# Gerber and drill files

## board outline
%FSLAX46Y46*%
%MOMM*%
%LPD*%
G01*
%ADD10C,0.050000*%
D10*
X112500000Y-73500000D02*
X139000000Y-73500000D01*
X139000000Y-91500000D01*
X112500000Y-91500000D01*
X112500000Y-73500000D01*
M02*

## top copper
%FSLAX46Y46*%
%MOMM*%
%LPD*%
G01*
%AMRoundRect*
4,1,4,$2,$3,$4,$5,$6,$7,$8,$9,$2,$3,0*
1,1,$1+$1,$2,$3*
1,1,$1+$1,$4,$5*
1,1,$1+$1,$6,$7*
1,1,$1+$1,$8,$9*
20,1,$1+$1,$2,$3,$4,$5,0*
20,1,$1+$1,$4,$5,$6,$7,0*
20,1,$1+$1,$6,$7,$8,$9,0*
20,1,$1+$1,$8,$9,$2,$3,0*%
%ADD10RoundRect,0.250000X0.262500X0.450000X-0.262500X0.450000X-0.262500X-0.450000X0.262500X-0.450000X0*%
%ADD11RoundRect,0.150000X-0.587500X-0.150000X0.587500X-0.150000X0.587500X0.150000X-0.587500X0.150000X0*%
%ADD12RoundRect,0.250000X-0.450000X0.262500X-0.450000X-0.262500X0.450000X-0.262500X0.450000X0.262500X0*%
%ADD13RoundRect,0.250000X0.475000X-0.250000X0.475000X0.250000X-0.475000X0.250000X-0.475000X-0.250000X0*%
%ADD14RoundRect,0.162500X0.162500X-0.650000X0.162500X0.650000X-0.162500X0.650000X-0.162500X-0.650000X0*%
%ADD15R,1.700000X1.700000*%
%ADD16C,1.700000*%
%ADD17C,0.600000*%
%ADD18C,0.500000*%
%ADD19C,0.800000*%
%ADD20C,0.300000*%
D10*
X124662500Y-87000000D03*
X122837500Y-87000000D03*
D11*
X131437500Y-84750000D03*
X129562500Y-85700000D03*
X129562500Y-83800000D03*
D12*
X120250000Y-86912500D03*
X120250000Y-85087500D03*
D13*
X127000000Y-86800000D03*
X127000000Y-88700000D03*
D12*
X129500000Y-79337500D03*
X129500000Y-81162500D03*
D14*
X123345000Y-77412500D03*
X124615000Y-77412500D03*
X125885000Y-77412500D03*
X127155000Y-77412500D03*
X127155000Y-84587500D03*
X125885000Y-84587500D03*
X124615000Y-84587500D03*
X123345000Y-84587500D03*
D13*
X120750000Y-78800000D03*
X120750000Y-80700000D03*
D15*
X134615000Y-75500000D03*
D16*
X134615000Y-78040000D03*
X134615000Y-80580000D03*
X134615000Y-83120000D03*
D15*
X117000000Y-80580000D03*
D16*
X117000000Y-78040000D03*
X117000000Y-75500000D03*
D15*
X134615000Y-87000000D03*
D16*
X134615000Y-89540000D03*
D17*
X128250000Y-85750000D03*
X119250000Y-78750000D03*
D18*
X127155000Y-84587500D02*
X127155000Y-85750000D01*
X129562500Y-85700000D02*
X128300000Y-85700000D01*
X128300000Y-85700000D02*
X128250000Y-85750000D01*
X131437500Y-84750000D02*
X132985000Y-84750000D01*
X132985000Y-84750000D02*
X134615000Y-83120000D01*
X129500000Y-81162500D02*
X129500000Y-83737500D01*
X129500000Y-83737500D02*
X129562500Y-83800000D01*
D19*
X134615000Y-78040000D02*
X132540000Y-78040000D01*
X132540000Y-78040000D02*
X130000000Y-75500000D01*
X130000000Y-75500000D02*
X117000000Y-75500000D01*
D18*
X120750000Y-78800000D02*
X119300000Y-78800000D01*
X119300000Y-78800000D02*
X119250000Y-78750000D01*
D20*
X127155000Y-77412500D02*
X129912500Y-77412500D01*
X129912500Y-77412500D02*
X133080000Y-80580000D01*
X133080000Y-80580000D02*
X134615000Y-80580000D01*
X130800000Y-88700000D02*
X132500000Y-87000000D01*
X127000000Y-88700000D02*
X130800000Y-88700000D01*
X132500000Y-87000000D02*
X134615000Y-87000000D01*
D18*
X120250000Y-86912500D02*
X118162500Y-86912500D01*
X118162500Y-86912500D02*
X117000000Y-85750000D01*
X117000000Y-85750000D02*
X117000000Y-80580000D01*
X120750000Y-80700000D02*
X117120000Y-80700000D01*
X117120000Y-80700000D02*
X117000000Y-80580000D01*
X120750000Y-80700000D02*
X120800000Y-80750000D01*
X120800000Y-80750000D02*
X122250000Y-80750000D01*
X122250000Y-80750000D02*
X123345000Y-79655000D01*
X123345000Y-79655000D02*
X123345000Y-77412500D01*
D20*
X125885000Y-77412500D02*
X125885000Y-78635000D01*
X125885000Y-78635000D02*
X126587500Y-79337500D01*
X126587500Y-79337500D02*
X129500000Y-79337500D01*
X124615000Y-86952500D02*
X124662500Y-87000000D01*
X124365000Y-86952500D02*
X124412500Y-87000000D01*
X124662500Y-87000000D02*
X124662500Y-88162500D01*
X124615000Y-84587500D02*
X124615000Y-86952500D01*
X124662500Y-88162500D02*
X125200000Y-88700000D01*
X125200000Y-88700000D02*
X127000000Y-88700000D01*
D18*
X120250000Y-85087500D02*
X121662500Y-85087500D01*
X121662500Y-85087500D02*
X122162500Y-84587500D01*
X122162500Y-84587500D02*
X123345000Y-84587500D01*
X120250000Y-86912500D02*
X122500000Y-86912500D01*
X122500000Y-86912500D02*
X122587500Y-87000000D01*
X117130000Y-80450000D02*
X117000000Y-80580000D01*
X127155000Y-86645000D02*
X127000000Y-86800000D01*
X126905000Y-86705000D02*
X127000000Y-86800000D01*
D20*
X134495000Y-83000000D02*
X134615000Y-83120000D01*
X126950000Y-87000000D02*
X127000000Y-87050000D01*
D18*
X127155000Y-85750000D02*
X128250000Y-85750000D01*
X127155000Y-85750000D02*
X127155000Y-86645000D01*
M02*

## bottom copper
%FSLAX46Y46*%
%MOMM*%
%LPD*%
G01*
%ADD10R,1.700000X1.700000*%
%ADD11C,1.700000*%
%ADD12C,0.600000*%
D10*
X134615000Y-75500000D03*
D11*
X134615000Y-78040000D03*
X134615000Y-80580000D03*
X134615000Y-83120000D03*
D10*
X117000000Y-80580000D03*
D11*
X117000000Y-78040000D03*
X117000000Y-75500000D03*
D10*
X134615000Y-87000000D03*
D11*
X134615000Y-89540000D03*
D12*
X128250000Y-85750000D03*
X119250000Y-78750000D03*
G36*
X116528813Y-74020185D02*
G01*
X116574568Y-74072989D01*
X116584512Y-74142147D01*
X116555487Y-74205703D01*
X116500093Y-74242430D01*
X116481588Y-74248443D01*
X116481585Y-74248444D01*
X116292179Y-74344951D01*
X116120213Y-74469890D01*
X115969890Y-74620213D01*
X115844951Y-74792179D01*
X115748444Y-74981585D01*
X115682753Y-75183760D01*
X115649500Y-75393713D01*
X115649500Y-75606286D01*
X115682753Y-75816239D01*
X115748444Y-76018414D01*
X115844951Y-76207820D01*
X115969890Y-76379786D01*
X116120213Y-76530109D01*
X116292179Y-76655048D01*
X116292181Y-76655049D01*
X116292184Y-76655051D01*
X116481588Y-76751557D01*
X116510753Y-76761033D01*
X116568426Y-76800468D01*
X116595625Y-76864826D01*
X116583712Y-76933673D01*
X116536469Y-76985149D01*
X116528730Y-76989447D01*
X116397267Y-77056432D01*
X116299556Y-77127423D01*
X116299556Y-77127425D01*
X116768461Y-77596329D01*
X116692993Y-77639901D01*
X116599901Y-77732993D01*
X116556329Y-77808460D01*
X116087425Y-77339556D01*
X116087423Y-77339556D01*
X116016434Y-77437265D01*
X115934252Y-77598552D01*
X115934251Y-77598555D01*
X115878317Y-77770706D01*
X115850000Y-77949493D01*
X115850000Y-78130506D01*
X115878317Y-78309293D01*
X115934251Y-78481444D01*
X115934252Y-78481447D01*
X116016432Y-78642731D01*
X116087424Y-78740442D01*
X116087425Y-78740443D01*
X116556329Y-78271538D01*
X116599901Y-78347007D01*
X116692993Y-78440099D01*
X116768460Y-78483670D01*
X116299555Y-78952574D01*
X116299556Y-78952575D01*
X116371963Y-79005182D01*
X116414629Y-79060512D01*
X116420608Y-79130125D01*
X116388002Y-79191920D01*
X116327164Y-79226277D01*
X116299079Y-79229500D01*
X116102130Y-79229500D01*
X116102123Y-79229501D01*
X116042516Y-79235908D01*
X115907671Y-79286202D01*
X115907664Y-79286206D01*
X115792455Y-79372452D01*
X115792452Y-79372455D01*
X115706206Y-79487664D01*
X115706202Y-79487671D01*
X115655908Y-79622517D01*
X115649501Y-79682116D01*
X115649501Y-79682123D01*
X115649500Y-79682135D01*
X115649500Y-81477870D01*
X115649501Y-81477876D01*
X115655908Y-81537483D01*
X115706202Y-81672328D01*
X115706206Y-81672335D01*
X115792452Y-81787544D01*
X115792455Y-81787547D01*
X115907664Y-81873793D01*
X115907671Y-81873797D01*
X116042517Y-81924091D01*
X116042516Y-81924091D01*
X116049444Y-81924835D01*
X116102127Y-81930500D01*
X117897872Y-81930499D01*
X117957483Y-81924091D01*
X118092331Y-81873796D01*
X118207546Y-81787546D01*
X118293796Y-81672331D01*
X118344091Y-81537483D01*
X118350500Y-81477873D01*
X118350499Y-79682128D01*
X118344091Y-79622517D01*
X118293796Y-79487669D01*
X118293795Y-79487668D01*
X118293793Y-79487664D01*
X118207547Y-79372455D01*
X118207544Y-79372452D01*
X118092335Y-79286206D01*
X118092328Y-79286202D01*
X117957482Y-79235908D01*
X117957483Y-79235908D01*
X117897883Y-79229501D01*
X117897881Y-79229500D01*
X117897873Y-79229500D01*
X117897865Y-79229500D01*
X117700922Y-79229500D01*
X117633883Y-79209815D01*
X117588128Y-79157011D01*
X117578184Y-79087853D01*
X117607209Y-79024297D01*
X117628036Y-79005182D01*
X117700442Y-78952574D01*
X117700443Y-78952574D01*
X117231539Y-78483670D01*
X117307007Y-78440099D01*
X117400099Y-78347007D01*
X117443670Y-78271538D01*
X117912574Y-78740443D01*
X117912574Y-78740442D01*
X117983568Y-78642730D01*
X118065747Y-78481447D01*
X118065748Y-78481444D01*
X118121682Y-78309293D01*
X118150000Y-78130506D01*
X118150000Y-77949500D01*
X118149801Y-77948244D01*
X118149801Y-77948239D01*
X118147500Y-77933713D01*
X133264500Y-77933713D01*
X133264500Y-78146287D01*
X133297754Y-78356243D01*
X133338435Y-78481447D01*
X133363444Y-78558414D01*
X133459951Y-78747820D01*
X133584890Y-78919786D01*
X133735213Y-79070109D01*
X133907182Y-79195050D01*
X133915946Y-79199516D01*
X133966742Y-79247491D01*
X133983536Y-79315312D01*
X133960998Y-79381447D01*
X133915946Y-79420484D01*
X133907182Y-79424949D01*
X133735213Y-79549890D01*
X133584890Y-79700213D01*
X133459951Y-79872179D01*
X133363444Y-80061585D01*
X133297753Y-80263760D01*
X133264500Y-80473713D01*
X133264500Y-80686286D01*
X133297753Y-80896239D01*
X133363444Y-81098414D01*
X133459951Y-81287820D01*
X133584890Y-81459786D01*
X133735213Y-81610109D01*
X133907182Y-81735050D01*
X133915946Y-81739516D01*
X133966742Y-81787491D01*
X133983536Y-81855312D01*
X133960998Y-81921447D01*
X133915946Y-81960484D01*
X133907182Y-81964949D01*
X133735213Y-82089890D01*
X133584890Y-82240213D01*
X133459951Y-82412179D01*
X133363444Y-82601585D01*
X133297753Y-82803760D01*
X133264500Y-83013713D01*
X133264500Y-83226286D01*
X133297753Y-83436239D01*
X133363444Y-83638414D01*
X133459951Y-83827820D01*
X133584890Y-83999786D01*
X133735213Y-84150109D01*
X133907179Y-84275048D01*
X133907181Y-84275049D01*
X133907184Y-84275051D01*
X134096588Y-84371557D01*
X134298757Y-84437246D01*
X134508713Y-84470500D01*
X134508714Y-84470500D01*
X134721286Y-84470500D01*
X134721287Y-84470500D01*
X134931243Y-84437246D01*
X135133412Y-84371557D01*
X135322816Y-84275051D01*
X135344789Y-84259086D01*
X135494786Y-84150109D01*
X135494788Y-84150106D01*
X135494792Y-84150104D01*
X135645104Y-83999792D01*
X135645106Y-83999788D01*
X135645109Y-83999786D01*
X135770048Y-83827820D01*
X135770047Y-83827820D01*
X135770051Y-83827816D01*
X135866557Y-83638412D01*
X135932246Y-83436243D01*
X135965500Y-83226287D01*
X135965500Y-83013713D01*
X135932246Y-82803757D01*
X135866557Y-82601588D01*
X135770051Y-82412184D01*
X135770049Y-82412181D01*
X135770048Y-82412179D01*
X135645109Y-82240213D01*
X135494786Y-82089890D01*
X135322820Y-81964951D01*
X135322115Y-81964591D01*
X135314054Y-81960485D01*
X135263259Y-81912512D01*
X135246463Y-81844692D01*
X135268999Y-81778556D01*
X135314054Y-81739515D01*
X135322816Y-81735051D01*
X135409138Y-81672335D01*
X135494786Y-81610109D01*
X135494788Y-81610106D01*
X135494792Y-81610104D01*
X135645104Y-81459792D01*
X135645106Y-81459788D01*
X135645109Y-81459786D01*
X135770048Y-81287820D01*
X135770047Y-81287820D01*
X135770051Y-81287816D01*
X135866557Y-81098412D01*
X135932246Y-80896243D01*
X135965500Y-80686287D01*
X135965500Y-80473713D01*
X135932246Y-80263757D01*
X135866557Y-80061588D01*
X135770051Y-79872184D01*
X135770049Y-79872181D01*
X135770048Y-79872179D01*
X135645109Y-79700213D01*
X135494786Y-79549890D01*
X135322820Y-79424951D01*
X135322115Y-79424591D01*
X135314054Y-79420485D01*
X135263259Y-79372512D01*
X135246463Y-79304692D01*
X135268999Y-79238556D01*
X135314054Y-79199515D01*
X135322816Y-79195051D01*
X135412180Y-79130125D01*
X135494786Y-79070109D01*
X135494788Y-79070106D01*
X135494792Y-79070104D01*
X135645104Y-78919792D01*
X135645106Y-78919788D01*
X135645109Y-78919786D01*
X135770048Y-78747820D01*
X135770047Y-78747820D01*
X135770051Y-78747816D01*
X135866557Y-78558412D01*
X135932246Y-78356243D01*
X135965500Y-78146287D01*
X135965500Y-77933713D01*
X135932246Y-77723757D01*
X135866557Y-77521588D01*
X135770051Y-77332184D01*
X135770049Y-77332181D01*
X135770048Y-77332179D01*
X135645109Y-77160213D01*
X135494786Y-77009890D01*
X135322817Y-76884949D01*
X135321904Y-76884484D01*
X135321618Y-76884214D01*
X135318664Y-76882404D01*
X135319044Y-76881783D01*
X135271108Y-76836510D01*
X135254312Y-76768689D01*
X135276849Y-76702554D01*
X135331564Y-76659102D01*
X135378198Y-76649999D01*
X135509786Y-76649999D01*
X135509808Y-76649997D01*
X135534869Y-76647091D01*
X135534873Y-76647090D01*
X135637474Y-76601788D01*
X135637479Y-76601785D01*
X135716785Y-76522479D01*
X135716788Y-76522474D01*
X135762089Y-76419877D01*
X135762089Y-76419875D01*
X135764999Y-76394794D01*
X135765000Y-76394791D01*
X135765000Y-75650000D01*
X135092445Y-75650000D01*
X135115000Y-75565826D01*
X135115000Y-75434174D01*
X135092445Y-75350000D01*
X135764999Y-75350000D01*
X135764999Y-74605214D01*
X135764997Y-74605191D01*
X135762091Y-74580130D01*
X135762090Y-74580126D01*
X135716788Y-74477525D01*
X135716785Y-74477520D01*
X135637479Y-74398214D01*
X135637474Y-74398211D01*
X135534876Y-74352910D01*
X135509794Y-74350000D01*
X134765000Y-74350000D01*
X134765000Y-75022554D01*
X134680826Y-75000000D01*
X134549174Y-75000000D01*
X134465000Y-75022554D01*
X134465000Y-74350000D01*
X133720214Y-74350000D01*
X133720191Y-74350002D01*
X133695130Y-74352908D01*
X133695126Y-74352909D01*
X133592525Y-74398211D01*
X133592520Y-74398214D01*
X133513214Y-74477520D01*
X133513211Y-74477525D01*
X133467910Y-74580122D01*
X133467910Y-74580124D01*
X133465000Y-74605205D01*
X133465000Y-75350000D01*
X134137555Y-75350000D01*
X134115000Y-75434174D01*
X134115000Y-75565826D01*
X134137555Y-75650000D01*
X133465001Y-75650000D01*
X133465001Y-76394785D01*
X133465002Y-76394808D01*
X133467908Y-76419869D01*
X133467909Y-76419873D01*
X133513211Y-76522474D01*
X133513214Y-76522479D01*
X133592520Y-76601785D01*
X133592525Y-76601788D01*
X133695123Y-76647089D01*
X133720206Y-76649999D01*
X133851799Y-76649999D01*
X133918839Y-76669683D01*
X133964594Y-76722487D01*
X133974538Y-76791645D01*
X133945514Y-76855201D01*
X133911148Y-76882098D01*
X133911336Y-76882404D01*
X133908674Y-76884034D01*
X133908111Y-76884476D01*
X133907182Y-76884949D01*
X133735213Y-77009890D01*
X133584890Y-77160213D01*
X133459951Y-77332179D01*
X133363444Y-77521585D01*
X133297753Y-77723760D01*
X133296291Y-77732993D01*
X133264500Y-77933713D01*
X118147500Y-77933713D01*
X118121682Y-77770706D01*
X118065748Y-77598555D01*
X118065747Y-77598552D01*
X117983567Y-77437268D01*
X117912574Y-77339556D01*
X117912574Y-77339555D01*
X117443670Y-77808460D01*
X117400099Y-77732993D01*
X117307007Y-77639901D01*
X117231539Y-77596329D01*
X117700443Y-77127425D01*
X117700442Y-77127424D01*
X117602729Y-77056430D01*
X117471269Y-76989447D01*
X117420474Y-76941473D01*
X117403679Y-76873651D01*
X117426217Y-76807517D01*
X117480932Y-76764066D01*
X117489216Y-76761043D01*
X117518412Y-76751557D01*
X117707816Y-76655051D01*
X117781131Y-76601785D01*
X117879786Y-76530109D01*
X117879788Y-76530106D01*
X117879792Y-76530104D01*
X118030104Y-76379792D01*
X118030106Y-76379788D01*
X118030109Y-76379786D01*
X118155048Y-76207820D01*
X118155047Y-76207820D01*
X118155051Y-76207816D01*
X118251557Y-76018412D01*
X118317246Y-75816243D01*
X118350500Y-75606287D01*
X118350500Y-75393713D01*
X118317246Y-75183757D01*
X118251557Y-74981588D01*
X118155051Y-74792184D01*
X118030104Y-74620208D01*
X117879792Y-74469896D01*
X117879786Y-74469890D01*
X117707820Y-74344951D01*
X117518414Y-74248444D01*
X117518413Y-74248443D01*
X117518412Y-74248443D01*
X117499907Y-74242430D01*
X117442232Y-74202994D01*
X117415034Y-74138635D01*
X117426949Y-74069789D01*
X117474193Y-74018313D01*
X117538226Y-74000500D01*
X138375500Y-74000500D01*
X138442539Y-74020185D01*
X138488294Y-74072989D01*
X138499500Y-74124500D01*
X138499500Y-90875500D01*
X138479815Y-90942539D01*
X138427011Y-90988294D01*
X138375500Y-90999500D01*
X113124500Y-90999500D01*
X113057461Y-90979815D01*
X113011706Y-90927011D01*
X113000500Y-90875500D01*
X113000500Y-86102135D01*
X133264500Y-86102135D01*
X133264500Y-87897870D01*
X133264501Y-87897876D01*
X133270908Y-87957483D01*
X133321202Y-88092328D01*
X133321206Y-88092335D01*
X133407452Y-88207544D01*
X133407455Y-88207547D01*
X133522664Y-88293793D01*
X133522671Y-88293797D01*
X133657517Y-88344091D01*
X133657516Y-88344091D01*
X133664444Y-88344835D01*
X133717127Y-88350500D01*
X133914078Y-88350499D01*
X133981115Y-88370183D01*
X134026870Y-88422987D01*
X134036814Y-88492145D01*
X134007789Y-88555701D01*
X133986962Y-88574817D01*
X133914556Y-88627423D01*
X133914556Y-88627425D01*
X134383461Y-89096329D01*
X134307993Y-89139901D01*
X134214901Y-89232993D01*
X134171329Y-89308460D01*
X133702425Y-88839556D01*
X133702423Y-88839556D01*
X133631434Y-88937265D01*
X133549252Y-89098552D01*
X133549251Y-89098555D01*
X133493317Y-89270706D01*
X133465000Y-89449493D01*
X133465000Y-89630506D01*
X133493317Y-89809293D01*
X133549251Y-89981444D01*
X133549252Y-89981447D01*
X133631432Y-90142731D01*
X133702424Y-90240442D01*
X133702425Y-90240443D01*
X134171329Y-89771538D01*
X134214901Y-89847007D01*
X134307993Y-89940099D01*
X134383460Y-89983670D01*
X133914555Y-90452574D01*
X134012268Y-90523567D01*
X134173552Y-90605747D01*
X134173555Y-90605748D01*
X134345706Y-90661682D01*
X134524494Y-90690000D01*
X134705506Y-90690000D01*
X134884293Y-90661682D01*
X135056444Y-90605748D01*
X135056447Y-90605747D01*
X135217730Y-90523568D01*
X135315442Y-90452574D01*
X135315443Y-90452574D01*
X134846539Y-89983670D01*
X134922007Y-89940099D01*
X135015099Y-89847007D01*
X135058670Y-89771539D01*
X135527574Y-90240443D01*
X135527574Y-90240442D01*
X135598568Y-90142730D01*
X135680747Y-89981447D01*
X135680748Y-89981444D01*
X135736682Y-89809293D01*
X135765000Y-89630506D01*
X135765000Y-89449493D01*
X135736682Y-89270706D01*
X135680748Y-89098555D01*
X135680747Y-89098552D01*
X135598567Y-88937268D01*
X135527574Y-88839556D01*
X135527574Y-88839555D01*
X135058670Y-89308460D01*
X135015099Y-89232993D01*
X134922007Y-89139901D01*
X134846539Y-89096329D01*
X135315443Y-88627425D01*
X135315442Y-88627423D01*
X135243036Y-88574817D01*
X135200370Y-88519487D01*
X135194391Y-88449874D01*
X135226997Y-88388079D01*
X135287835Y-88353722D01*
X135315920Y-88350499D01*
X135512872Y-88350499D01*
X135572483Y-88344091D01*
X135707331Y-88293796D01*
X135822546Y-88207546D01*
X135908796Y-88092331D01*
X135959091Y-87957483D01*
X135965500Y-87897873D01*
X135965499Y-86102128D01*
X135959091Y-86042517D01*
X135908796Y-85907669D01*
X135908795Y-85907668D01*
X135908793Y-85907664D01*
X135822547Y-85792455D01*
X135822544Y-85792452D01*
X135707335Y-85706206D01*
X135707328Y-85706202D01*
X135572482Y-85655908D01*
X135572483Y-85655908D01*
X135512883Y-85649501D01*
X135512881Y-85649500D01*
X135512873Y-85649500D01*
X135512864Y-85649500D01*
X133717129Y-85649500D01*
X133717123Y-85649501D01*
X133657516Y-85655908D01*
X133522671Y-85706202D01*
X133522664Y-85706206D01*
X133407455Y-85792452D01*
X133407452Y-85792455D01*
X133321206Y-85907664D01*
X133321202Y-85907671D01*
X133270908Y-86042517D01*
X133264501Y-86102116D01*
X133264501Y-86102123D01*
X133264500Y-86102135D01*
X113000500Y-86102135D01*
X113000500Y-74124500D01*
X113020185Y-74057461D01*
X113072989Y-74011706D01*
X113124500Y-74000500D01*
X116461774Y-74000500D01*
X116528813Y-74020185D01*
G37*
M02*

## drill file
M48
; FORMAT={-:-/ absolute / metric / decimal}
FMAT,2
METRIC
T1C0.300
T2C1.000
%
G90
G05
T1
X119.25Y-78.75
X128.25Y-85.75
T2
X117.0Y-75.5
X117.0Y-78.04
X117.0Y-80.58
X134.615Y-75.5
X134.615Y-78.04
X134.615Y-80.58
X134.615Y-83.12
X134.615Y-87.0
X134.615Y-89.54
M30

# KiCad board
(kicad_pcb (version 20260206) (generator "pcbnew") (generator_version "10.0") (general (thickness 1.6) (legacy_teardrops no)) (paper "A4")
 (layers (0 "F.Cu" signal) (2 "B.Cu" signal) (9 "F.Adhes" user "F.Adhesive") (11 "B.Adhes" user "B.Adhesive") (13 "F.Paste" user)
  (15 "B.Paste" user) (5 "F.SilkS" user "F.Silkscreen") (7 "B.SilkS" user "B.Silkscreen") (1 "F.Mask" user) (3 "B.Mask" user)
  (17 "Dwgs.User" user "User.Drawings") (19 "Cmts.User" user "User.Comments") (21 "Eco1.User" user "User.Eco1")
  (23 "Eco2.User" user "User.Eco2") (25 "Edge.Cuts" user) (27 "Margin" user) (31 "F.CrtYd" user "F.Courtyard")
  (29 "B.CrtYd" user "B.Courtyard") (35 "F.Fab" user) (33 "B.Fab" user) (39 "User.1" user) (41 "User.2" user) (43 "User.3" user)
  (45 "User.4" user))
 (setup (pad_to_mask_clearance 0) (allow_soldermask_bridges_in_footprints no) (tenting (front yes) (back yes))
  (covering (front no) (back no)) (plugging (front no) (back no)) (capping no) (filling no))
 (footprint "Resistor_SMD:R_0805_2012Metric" (layer "F.Cu") (at 123.75 87 180)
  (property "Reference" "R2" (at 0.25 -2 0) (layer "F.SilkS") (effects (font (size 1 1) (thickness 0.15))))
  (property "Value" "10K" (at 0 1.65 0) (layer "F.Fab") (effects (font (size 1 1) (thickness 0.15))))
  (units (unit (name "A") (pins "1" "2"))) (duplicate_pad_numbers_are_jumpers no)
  (pad "1" smd roundrect (at -0.9125 0 180) (size 1.025 1.4) (layers "F.Cu" "F.Mask" "F.Paste") (roundrect_rratio 0.243902)
   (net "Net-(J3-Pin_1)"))
  (pad "2" smd roundrect (at 0.9125 0 180) (size 1.025 1.4) (layers "F.Cu" "F.Mask" "F.Paste") (roundrect_rratio 0.243902) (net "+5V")))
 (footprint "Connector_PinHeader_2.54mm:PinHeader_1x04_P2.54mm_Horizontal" (layer "F.Cu") (at 134.615 75.5)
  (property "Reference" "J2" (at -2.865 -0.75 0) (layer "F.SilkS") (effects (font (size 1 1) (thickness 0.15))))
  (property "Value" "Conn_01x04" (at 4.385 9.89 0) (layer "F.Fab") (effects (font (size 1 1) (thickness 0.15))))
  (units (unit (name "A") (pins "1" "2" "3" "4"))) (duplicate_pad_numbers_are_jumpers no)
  (pad "1" thru_hole rect (at 0 0) (size 1.7 1.7) (drill 1) (layers "*.Cu" "*.Mask") (remove_unused_layers no) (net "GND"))
  (pad "2" thru_hole circle (at 0 2.54) (size 1.7 1.7) (drill 1) (layers "*.Cu" "*.Mask") (remove_unused_layers no) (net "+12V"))
  (pad "3" thru_hole circle (at 0 5.08) (size 1.7 1.7) (drill 1) (layers "*.Cu" "*.Mask") (remove_unused_layers no) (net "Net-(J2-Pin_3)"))
  (pad "4" thru_hole circle (at 0 7.62) (size 1.7 1.7) (drill 1) (layers "*.Cu" "*.Mask") (remove_unused_layers no) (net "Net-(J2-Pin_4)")))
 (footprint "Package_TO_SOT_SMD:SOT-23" (layer "F.Cu") (at 130.5 84.75)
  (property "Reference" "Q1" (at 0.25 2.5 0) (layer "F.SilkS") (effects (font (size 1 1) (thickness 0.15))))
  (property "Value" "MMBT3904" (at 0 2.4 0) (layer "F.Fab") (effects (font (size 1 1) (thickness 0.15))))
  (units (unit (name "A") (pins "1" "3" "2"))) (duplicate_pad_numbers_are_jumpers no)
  (pad "1" smd roundrect (at -0.9375 -0.95) (size 1.475 0.6) (layers "F.Cu" "F.Mask" "F.Paste") (roundrect_rratio 0.25) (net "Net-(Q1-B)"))
  (pad "2" smd roundrect (at -0.9375 0.95) (size 1.475 0.6) (layers "F.Cu" "F.Mask" "F.Paste") (roundrect_rratio 0.25) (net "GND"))
  (pad "3" smd roundrect (at 0.9375 0) (size 1.475 0.6) (layers "F.Cu" "F.Mask" "F.Paste") (roundrect_rratio 0.25) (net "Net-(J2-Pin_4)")))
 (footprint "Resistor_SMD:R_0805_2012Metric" (layer "F.Cu") (at 120.25 86 -90)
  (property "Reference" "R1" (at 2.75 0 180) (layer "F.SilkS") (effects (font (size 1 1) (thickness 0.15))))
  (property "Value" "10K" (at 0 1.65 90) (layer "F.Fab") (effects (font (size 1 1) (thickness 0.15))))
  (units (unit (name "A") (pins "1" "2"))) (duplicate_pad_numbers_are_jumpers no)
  (pad "1" smd roundrect (at -0.9125 0 270) (size 1.025 1.4) (layers "F.Cu" "F.Mask" "F.Paste") (roundrect_rratio 0.243902)
   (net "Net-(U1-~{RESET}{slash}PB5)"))
  (pad "2" smd roundrect (at 0.9125 0 270) (size 1.025 1.4) (layers "F.Cu" "F.Mask" "F.Paste") (roundrect_rratio 0.243902) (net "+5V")))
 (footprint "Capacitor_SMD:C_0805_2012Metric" (layer "F.Cu") (at 127 87.75 90)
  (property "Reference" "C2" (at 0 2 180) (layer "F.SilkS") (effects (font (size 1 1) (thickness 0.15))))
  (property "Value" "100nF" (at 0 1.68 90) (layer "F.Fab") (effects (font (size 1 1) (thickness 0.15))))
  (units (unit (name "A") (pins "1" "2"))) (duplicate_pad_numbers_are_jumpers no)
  (pad "1" smd roundrect (at -0.95 0 90) (size 1 1.45) (layers "F.Cu" "F.Mask" "F.Paste") (roundrect_rratio 0.25) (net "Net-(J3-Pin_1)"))
  (pad "2" smd roundrect (at 0.95 0 90) (size 1 1.45) (layers "F.Cu" "F.Mask" "F.Paste") (roundrect_rratio 0.25) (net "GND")))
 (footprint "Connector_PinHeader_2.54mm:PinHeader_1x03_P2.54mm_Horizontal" (layer "F.Cu") (at 117 80.58 180)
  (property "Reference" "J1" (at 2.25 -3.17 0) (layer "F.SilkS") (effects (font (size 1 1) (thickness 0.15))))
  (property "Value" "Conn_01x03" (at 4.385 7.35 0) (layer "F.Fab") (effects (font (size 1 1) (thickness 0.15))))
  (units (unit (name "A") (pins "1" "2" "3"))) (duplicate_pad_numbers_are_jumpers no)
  (pad "1" thru_hole rect (at 0 0 180) (size 1.7 1.7) (drill 1) (layers "*.Cu" "*.Mask") (remove_unused_layers no) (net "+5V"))
  (pad "2" thru_hole circle (at 0 2.54 180) (size 1.7 1.7) (drill 1) (layers "*.Cu" "*.Mask") (remove_unused_layers no) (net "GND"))
  (pad "3" thru_hole circle (at 0 5.08 180) (size 1.7 1.7) (drill 1) (layers "*.Cu" "*.Mask") (remove_unused_layers no) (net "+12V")))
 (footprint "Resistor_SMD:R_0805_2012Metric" (layer "F.Cu") (at 129.5 80.25 -90)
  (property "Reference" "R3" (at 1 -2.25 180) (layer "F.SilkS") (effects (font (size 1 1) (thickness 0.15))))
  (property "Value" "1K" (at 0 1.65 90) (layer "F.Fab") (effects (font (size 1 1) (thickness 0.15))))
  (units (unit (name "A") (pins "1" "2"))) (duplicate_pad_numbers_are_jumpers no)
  (pad "1" smd roundrect (at -0.9125 0 270) (size 1.025 1.4) (layers "F.Cu" "F.Mask" "F.Paste") (roundrect_rratio 0.243902)
   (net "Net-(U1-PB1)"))
  (pad "2" smd roundrect (at 0.9125 0 270) (size 1.025 1.4) (layers "F.Cu" "F.Mask" "F.Paste") (roundrect_rratio 0.243902)
   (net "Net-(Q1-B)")))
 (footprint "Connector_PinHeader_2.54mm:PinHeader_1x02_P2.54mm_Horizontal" (layer "F.Cu") (at 134.615 87)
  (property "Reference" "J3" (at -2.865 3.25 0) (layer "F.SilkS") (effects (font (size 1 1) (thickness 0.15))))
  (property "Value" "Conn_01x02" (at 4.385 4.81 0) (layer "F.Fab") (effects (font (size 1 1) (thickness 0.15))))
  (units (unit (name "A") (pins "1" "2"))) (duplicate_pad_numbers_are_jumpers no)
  (pad "1" thru_hole rect (at 0 0) (size 1.7 1.7) (drill 1) (layers "*.Cu" "*.Mask") (remove_unused_layers no) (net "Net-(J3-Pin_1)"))
  (pad "2" thru_hole circle (at 0 2.54) (size 1.7 1.7) (drill 1) (layers "*.Cu" "*.Mask") (remove_unused_layers no) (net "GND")))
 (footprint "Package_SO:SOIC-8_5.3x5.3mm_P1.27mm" (layer "F.Cu") (at 125.25 81 90)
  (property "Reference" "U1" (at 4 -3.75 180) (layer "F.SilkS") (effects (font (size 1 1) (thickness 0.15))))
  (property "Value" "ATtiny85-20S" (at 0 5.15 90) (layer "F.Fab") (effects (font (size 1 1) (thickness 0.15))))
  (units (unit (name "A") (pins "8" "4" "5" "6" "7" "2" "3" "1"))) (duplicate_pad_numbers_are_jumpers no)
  (pad "1" smd roundrect (at -3.5875 -1.905 90) (size 1.625 0.65) (layers "F.Cu" "F.Mask" "F.Paste") (roundrect_rratio 0.25)
   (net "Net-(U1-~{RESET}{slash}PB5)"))
  (pad "2" smd roundrect (at -3.5875 -0.635 90) (size 1.625 0.65) (layers "F.Cu" "F.Mask" "F.Paste") (roundrect_rratio 0.25)
   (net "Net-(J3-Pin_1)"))
  (pad "3" smd roundrect (at -3.5875 0.635 90) (size 1.625 0.65) (layers "F.Cu" "F.Mask" "F.Paste") (roundrect_rratio 0.25)
   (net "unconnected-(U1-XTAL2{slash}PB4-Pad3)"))
  (pad "4" smd roundrect (at -3.5875 1.905 90) (size 1.625 0.65) (layers "F.Cu" "F.Mask" "F.Paste") (roundrect_rratio 0.25) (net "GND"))
  (pad "5" smd roundrect (at 3.5875 1.905 90) (size 1.625 0.65) (layers "F.Cu" "F.Mask" "F.Paste") (roundrect_rratio 0.25)
   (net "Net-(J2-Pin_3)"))
  (pad "6" smd roundrect (at 3.5875 0.635 90) (size 1.625 0.65) (layers "F.Cu" "F.Mask" "F.Paste") (roundrect_rratio 0.25)
   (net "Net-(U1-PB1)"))
  (pad "7" smd roundrect (at 3.5875 -0.635 90) (size 1.625 0.65) (layers "F.Cu" "F.Mask" "F.Paste") (roundrect_rratio 0.25)
   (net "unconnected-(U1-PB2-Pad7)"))
  (pad "8" smd roundrect (at 3.5875 -1.905 90) (size 1.625 0.65) (layers "F.Cu" "F.Mask" "F.Paste") (roundrect_rratio 0.25) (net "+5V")))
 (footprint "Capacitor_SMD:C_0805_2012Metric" (layer "F.Cu") (at 120.75 79.75 90)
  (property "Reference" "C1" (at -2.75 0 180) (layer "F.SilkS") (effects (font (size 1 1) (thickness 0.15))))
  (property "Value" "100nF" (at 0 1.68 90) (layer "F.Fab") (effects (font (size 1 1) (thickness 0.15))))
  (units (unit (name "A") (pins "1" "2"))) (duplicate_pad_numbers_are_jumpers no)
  (pad "1" smd roundrect (at -0.95 0 90) (size 1 1.45) (layers "F.Cu" "F.Mask" "F.Paste") (roundrect_rratio 0.25) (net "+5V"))
  (pad "2" smd roundrect (at 0.95 0 90) (size 1 1.45) (layers "F.Cu" "F.Mask" "F.Paste") (roundrect_rratio 0.25) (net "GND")))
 (gr_rect (start 112.5 73.5) (end 139 91.5) (stroke (width 0.05) (type default)) (fill no) (layer "Edge.Cuts"))
 (segment (start 124.6625 87) (end 124.6625 88.1625) (width 0.3) (layer "F.Cu") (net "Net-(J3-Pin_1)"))
 (segment (start 132.5 87) (end 134.615 87) (width 0.3) (layer "F.Cu") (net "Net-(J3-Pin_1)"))
 (segment (start 124.365 86.9525) (end 124.4125 87) (width 0.3) (layer "F.Cu") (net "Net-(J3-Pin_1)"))
 (segment (start 130.8 88.7) (end 132.5 87) (width 0.3) (layer "F.Cu") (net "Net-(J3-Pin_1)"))
 (segment (start 127 88.7) (end 130.8 88.7) (width 0.3) (layer "F.Cu") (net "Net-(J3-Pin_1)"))
 (segment (start 125.2 88.7) (end 127 88.7) (width 0.3) (layer "F.Cu") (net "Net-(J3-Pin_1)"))
 (segment (start 124.615 86.9525) (end 124.6625 87) (width 0.3) (layer "F.Cu") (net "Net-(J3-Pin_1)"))
 (segment (start 124.615 84.5875) (end 124.615 86.9525) (width 0.3) (layer "F.Cu") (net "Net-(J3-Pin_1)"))
 (segment (start 124.6625 88.1625) (end 125.2 88.7) (width 0.3) (layer "F.Cu") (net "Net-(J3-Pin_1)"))
 (segment (start 117 85.75) (end 117 80.58) (width 0.5) (layer "F.Cu") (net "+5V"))
 (segment (start 120.8 80.75) (end 122.25 80.75) (width 0.5) (layer "F.Cu") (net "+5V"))
 (segment (start 117.12 80.7) (end 117 80.58) (width 0.5) (layer "F.Cu") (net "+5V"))
 (segment (start 122.5 86.9125) (end 122.5875 87) (width 0.5) (layer "F.Cu") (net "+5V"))
 (segment (start 120.25 86.9125) (end 118.1625 86.9125) (width 0.5) (layer "F.Cu") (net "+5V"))
 (segment (start 120.75 80.7) (end 120.8 80.75) (width 0.5) (layer "F.Cu") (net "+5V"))
 (segment (start 117.13 80.45) (end 117 80.58) (width 0.5) (layer "F.Cu") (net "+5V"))
 (segment (start 122.25 80.75) (end 123.345 79.655) (width 0.5) (layer "F.Cu") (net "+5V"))
 (segment (start 123.345 79.655) (end 123.345 77.4125) (width 0.5) (layer "F.Cu") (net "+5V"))
 (segment (start 120.25 86.9125) (end 122.5 86.9125) (width 0.5) (layer "F.Cu") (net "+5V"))
 (segment (start 118.1625 86.9125) (end 117 85.75) (width 0.5) (layer "F.Cu") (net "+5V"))
 (segment (start 120.75 80.7) (end 117.12 80.7) (width 0.5) (layer "F.Cu") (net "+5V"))
 (segment (start 127.155 85.75) (end 127.155 86.645) (width 0.5) (layer "F.Cu") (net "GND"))
 (segment (start 126.95 87) (end 127 87.05) (width 0.3) (layer "F.Cu") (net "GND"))
 (segment (start 127.155 86.645) (end 127 86.8) (width 0.5) (layer "F.Cu") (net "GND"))
 (segment (start 119.3 78.8) (end 119.25 78.75) (width 0.5) (layer "F.Cu") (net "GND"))
 (segment (start 128.3 85.7) (end 128.25 85.75) (width 0.5) (layer "F.Cu") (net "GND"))
 (segment (start 129.5625 85.7) (end 128.3 85.7) (width 0.5) (layer "F.Cu") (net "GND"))
 (segment (start 127.155 85.75) (end 128.25 85.75) (width 0.5) (layer "F.Cu") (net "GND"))
 (segment (start 127.155 84.5875) (end 127.155 85.75) (width 0.5) (layer "F.Cu") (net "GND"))
 (segment (start 126.905 86.705) (end 127 86.8) (width 0.5) (layer "F.Cu") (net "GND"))
 (segment (start 120.75 78.8) (end 119.3 78.8) (width 0.5) (layer "F.Cu") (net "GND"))
 (via (at 128.25 85.75) (size 0.6) (drill 0.3) (layers "F.Cu" "B.Cu") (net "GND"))
 (via (at 119.25 78.75) (size 0.6) (drill 0.3) (layers "F.Cu" "B.Cu") (free yes) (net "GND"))
 (segment (start 130 75.5) (end 117 75.5) (width 0.8) (layer "F.Cu") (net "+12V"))
 (segment (start 132.54 78.04) (end 130 75.5) (width 0.8) (layer "F.Cu") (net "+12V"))
 (segment (start 134.615 78.04) (end 132.54 78.04) (width 0.8) (layer "F.Cu") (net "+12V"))
 (segment (start 127.155 77.4125) (end 129.9125 77.4125) (width 0.3) (layer "F.Cu") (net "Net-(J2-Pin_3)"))
 (segment (start 129.9125 77.4125) (end 133.08 80.58) (width 0.3) (layer "F.Cu") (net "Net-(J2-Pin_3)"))
 (segment (start 133.08 80.58) (end 134.615 80.58) (width 0.3) (layer "F.Cu") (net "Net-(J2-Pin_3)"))
 (segment (start 131.4375 84.75) (end 132.985 84.75) (width 0.5) (layer "F.Cu") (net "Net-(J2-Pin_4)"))
 (segment (start 134.495 83) (end 134.615 83.12) (width 0.3) (layer "F.Cu") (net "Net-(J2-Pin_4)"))
 (segment (start 132.985 84.75) (end 134.615 83.12) (width 0.5) (layer "F.Cu") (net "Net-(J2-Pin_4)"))
 (segment (start 129.5 83.7375) (end 129.5625 83.8) (width 0.5) (layer "F.Cu") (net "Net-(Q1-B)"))
 (segment (start 129.5 81.1625) (end 129.5 83.7375) (width 0.5) (layer "F.Cu") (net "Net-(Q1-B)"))
 (segment (start 122.1625 84.5875) (end 123.345 84.5875) (width 0.5) (layer "F.Cu") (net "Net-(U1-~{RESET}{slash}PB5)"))
 (segment (start 121.6625 85.0875) (end 122.1625 84.5875) (width 0.5) (layer "F.Cu") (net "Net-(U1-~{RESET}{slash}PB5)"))
 (segment (start 120.25 85.0875) (end 121.6625 85.0875) (width 0.5) (layer "F.Cu") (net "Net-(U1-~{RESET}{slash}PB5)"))
 (segment (start 126.5875 79.3375) (end 129.5 79.3375) (width 0.3) (layer "F.Cu") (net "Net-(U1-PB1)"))
 (segment (start 125.885 77.4125) (end 125.885 78.635) (width 0.3) (layer "F.Cu") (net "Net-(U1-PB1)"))
 (segment (start 125.885 78.635) (end 126.5875 79.3375) (width 0.3) (layer "F.Cu") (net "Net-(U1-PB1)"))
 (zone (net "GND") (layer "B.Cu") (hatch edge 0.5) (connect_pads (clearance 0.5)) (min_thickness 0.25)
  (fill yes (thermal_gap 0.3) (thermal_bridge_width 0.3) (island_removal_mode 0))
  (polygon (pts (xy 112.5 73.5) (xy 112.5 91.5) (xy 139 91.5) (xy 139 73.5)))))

